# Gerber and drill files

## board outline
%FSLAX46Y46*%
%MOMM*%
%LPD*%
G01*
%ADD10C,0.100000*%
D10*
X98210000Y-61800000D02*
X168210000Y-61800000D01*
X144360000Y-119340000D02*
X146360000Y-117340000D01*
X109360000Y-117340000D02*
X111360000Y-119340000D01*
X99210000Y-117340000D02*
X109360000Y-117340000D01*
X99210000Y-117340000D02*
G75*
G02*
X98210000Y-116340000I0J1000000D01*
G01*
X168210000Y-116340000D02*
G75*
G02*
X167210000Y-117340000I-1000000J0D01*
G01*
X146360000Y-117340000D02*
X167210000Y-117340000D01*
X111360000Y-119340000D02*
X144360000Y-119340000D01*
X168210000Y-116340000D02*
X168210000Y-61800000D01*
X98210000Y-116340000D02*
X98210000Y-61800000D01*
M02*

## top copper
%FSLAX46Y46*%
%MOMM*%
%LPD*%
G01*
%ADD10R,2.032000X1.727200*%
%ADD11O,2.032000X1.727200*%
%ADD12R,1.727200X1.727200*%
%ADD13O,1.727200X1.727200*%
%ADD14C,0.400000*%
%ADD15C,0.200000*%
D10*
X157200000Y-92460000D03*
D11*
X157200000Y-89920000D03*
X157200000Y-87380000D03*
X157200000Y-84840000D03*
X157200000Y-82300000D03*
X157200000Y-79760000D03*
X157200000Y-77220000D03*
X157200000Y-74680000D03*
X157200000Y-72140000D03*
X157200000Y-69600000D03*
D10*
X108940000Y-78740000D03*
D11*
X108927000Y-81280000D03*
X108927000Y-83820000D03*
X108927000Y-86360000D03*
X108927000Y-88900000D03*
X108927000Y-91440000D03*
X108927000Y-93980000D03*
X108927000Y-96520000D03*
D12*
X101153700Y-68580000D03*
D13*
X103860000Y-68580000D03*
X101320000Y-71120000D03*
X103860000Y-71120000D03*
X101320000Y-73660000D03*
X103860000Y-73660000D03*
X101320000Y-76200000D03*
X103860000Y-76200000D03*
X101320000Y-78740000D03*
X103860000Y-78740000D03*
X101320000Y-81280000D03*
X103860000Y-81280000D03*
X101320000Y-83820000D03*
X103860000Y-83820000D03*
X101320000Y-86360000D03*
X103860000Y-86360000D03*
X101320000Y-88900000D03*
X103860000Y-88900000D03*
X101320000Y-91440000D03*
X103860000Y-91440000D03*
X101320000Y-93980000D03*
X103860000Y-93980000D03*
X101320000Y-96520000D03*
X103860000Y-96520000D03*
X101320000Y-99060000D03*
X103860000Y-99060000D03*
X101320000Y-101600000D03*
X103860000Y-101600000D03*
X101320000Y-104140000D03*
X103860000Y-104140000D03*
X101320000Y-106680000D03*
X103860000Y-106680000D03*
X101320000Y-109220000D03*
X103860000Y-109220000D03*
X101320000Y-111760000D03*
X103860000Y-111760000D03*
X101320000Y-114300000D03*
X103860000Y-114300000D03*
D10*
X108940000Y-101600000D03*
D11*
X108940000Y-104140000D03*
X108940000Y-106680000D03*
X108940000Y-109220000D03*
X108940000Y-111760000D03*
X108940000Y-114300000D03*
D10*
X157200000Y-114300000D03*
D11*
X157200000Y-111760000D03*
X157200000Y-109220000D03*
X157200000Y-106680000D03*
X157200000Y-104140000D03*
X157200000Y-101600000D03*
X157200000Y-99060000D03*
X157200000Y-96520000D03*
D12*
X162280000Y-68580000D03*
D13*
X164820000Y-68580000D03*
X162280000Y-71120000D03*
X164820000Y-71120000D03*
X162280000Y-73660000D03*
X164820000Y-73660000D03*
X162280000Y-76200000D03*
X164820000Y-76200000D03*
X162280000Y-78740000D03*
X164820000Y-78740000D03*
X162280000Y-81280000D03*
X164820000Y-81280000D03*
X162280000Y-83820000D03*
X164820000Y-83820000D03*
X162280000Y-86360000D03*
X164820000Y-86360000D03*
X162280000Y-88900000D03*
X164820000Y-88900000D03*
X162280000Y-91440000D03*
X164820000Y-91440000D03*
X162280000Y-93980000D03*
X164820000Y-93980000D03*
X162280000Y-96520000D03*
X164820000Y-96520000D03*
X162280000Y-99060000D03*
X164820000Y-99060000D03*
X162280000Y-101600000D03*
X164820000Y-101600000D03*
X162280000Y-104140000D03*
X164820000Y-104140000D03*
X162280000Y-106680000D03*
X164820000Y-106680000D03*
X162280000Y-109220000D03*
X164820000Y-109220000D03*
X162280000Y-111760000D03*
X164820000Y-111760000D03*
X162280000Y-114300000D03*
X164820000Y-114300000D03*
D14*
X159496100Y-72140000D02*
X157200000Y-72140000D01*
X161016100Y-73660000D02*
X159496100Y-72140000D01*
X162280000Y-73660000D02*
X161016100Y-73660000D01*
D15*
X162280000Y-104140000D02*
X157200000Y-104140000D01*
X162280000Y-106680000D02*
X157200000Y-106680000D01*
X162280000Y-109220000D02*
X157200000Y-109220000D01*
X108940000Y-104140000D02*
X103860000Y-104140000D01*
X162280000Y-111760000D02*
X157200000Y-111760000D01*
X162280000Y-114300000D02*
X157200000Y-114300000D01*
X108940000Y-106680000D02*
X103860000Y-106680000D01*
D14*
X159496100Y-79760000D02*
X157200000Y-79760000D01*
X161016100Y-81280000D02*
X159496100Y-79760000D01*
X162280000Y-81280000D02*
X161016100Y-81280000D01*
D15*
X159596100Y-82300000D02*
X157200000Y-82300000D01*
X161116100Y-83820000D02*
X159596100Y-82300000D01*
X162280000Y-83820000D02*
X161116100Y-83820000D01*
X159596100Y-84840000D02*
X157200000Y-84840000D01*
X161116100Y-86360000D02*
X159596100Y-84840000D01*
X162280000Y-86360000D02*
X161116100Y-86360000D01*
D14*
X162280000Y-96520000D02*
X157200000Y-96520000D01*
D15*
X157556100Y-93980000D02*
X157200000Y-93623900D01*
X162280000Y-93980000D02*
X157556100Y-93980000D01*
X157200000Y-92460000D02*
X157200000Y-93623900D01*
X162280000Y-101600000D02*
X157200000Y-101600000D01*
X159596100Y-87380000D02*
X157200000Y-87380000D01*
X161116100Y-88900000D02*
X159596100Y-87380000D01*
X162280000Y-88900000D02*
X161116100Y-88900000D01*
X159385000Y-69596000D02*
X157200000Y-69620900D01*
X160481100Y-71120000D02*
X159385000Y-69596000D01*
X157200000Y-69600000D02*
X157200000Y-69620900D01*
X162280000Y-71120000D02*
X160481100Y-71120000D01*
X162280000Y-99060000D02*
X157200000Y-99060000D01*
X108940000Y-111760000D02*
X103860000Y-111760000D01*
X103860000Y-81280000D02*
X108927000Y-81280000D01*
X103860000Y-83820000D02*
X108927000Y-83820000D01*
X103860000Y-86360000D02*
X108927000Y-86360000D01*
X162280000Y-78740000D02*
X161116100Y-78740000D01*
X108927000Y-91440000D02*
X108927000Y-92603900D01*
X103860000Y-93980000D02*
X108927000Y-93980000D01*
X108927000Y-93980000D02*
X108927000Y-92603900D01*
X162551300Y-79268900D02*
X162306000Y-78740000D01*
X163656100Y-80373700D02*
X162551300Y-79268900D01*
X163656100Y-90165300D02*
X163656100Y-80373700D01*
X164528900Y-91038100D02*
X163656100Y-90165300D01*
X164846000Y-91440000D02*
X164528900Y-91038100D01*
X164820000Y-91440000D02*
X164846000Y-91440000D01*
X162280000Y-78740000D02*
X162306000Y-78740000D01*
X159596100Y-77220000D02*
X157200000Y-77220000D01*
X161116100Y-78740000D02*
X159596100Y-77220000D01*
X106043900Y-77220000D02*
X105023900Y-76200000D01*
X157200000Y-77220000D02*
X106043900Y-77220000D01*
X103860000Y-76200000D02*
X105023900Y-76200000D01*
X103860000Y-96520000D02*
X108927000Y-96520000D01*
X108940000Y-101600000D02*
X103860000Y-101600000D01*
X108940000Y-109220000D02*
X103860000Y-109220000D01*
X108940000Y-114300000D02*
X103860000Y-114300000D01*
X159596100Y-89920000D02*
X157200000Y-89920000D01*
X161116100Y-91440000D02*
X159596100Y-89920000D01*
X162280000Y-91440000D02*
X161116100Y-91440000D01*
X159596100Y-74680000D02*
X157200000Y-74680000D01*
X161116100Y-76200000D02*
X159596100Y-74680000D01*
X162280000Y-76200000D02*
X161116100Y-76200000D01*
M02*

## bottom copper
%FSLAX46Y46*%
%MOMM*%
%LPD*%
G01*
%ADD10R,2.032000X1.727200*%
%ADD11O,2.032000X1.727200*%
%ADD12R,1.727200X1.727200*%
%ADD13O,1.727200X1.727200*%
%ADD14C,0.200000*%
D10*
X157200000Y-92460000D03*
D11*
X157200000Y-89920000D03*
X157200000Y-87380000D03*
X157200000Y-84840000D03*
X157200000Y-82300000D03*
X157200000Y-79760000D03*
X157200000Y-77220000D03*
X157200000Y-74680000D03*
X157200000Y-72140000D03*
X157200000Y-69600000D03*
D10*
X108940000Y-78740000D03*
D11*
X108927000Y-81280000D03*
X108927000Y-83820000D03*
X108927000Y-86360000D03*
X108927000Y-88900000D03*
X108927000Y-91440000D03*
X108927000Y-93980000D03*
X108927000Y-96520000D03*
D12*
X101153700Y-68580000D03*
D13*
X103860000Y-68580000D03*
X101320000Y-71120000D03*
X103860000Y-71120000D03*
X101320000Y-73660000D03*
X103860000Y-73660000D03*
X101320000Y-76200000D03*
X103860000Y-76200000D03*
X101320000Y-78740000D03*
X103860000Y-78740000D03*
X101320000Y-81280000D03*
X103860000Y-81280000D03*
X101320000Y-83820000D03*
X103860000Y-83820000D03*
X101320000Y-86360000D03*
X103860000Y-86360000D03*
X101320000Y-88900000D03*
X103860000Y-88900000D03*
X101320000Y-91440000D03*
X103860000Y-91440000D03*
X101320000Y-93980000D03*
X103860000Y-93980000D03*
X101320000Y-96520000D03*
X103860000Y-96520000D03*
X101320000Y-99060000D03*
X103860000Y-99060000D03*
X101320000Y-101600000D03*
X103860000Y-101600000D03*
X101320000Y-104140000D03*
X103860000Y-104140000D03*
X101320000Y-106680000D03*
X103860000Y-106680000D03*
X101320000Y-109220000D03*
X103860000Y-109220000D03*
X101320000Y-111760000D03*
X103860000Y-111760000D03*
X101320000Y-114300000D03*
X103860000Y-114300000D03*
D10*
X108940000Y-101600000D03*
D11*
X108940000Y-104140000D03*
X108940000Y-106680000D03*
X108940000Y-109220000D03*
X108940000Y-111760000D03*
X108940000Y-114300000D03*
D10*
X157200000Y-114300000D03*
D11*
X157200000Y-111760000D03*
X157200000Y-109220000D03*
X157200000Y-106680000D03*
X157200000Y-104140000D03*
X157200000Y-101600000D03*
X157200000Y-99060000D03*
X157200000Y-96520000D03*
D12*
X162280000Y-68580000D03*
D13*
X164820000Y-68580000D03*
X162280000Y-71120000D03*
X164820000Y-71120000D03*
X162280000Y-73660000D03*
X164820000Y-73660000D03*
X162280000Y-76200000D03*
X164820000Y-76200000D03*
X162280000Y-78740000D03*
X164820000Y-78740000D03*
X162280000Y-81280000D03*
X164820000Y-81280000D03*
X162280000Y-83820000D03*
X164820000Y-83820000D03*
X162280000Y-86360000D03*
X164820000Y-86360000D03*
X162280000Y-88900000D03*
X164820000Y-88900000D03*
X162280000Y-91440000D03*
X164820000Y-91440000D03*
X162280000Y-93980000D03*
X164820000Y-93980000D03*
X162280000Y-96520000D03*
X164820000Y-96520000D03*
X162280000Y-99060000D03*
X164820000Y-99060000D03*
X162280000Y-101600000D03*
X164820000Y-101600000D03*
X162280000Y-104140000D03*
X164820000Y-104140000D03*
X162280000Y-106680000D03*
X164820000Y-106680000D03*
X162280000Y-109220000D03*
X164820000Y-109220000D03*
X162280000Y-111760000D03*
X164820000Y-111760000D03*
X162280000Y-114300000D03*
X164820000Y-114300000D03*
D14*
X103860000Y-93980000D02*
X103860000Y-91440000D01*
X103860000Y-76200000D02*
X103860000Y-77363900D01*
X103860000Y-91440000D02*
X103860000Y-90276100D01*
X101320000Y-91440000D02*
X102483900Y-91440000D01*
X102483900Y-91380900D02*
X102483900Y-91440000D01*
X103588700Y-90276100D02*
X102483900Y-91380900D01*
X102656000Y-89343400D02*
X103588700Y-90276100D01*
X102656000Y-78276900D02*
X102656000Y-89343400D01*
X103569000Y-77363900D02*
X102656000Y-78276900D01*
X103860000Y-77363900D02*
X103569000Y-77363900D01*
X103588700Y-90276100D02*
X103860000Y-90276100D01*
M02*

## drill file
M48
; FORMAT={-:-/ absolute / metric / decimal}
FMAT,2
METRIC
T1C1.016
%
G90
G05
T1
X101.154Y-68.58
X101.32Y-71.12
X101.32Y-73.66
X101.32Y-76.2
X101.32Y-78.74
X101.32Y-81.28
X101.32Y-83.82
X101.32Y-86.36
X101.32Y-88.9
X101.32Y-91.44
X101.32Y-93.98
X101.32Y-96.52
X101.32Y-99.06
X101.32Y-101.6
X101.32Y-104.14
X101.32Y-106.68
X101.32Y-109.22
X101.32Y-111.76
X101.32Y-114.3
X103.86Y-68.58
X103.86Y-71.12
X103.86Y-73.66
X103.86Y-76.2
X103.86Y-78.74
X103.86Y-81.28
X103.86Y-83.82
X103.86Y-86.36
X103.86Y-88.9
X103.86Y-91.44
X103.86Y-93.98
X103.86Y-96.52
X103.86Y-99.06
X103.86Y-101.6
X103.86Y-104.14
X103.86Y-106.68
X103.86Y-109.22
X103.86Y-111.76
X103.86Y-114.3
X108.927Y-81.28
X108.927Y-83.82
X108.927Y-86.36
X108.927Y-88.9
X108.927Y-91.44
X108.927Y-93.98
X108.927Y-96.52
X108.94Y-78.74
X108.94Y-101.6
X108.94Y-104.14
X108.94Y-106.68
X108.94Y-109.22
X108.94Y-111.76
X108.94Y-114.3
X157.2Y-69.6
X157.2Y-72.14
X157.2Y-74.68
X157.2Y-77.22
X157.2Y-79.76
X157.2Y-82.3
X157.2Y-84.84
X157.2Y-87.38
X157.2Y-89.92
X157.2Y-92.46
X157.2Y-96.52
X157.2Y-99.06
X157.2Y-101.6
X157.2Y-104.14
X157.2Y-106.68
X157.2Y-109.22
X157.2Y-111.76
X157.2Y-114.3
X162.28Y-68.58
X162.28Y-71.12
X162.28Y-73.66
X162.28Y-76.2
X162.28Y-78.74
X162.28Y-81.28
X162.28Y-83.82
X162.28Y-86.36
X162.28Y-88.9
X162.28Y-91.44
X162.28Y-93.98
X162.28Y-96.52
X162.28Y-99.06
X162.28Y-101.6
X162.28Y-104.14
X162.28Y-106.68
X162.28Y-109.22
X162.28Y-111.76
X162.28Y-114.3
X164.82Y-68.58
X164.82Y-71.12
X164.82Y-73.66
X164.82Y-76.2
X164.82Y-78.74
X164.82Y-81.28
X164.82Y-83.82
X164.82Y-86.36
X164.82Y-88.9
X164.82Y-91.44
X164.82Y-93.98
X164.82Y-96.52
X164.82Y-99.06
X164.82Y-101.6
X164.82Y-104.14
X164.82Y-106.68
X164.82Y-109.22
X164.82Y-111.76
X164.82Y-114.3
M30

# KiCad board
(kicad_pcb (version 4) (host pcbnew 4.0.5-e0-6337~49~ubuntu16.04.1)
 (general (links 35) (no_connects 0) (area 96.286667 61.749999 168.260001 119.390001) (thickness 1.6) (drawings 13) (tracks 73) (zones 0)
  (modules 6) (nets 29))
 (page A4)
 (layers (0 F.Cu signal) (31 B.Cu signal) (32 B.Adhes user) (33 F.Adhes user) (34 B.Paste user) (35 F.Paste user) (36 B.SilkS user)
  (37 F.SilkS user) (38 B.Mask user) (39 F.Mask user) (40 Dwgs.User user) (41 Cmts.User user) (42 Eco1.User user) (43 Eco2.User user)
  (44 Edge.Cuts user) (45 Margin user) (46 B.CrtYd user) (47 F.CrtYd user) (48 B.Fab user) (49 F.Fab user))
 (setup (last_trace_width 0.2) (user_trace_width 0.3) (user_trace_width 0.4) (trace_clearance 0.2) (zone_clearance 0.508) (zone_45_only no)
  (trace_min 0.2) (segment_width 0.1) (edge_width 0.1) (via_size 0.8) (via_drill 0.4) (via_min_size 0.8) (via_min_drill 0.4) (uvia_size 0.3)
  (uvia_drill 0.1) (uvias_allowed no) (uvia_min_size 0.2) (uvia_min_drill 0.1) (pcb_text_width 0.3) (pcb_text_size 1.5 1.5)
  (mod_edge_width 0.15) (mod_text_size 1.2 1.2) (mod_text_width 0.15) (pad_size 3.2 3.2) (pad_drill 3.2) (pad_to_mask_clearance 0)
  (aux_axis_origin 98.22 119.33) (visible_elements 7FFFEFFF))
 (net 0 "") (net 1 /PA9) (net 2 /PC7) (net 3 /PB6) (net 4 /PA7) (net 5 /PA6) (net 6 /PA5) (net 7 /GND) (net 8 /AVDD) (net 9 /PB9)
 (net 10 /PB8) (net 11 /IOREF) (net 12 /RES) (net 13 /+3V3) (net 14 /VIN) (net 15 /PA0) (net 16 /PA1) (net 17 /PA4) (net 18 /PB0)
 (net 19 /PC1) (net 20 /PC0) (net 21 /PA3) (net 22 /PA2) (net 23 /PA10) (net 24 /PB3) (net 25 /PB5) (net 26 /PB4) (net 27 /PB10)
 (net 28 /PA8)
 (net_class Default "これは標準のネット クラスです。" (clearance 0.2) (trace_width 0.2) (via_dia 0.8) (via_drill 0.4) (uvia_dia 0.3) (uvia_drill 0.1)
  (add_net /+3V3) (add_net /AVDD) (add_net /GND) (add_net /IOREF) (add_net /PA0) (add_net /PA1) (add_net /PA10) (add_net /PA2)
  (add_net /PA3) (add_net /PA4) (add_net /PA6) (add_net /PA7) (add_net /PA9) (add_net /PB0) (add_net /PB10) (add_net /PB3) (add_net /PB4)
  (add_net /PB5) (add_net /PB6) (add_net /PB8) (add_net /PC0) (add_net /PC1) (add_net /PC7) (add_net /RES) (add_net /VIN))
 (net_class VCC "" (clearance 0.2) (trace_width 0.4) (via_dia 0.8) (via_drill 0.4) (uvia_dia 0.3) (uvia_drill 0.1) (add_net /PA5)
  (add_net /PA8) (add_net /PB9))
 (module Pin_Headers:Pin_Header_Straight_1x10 (layer F.Cu) (at 157.2 92.46 180)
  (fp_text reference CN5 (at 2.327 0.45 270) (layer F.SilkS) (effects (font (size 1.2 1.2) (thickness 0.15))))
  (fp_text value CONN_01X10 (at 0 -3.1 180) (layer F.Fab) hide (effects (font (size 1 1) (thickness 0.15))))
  (pad 1 thru_hole rect (at 0 0 180) (size 2.032 1.7272) (drill 1.016) (layers *.Cu *.Mask F.SilkS) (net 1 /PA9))
  (pad 2 thru_hole oval (at 0 2.54 180) (size 2.032 1.7272) (drill 1.016) (layers *.Cu *.Mask F.SilkS) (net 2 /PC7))
  (pad 3 thru_hole oval (at 0 5.08 180) (size 2.032 1.7272) (drill 1.016) (layers *.Cu *.Mask F.SilkS) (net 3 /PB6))
  (pad 4 thru_hole oval (at 0 7.62 180) (size 2.032 1.7272) (drill 1.016) (layers *.Cu *.Mask F.SilkS) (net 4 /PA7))
  (pad 5 thru_hole oval (at 0 10.16 180) (size 2.032 1.7272) (drill 1.016) (layers *.Cu *.Mask F.SilkS) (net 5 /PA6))
  (pad 6 thru_hole oval (at 0 12.7 180) (size 2.032 1.7272) (drill 1.016) (layers *.Cu *.Mask F.SilkS) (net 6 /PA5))
  (pad 7 thru_hole oval (at 0 15.24 180) (size 2.032 1.7272) (drill 1.016) (layers *.Cu *.Mask F.SilkS) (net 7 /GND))
  (pad 8 thru_hole oval (at 0 17.78 180) (size 2.032 1.7272) (drill 1.016) (layers *.Cu *.Mask F.SilkS) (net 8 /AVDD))
  (pad 9 thru_hole oval (at 0 20.32 180) (size 2.032 1.7272) (drill 1.016) (layers *.Cu *.Mask F.SilkS) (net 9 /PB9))
  (pad 10 thru_hole oval (at 0 22.86 180) (size 2.032 1.7272) (drill 1.016) (layers *.Cu *.Mask F.SilkS) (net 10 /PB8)))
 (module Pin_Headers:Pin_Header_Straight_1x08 (layer F.Cu) (at 108.927 78.74)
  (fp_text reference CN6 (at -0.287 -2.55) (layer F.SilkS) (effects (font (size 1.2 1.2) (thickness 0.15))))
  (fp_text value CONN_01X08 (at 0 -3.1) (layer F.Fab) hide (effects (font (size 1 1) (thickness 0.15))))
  (pad 1 thru_hole rect (at 0.013 0) (size 2.032 1.7272) (drill 1.016) (layers *.Cu *.Mask F.SilkS))
  (pad 2 thru_hole oval (at 0 2.54) (size 2.032 1.7272) (drill 1.016) (layers *.Cu *.Mask F.SilkS) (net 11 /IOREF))
  (pad 3 thru_hole oval (at 0 5.08) (size 2.032 1.7272) (drill 1.016) (layers *.Cu *.Mask F.SilkS) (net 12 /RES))
  (pad 4 thru_hole oval (at 0 7.62) (size 2.032 1.7272) (drill 1.016) (layers *.Cu *.Mask F.SilkS) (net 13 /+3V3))
  (pad 5 thru_hole oval (at 0 10.16) (size 2.032 1.7272) (drill 1.016) (layers *.Cu *.Mask F.SilkS))
  (pad 6 thru_hole oval (at 0 12.7) (size 2.032 1.7272) (drill 1.016) (layers *.Cu *.Mask F.SilkS) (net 7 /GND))
  (pad 7 thru_hole oval (at 0 15.24) (size 2.032 1.7272) (drill 1.016) (layers *.Cu *.Mask F.SilkS) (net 7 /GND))
  (pad 8 thru_hole oval (at 0 17.78) (size 2.032 1.7272) (drill 1.016) (layers *.Cu *.Mask F.SilkS) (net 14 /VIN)))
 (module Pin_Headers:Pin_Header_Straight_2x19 (layer F.Cu) (at 101.32 68.58)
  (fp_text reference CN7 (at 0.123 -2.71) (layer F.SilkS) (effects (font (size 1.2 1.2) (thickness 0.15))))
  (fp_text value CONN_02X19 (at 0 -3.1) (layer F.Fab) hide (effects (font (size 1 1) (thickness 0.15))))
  (pad 1 thru_hole rect (at -0.1663 0) (size 1.7272 1.7272) (drill 1.016) (layers *.Cu *.Mask F.SilkS))
  (pad 2 thru_hole oval (at 2.54 0) (size 1.7272 1.7272) (drill 1.016) (layers *.Cu *.Mask F.SilkS))
  (pad 3 thru_hole oval (at 0 2.54) (size 1.7272 1.7272) (drill 1.016) (layers *.Cu *.Mask F.SilkS))
  (pad 4 thru_hole oval (at 2.54 2.54) (size 1.7272 1.7272) (drill 1.016) (layers *.Cu *.Mask F.SilkS))
  (pad 5 thru_hole oval (at 0 5.08) (size 1.7272 1.7272) (drill 1.016) (layers *.Cu *.Mask F.SilkS))
  (pad 6 thru_hole oval (at 2.54 5.08) (size 1.7272 1.7272) (drill 1.016) (layers *.Cu *.Mask F.SilkS))
  (pad 7 thru_hole oval (at 0 7.62) (size 1.7272 1.7272) (drill 1.016) (layers *.Cu *.Mask F.SilkS))
  (pad 8 thru_hole oval (at 2.54 7.62) (size 1.7272 1.7272) (drill 1.016) (layers *.Cu *.Mask F.SilkS) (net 7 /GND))
  (pad 9 thru_hole oval (at 0 10.16) (size 1.7272 1.7272) (drill 1.016) (layers *.Cu *.Mask F.SilkS))
  (pad 10 thru_hole oval (at 2.54 10.16) (size 1.7272 1.7272) (drill 1.016) (layers *.Cu *.Mask F.SilkS))
  (pad 11 thru_hole oval (at 0 12.7) (size 1.7272 1.7272) (drill 1.016) (layers *.Cu *.Mask F.SilkS))
  (pad 12 thru_hole oval (at 2.54 12.7) (size 1.7272 1.7272) (drill 1.016) (layers *.Cu *.Mask F.SilkS) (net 11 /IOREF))
  (pad 13 thru_hole oval (at 0 15.24) (size 1.7272 1.7272) (drill 1.016) (layers *.Cu *.Mask F.SilkS))
  (pad 14 thru_hole oval (at 2.54 15.24) (size 1.7272 1.7272) (drill 1.016) (layers *.Cu *.Mask F.SilkS) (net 12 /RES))
  (pad 15 thru_hole oval (at 0 17.78) (size 1.7272 1.7272) (drill 1.016) (layers *.Cu *.Mask F.SilkS))
  (pad 16 thru_hole oval (at 2.54 17.78) (size 1.7272 1.7272) (drill 1.016) (layers *.Cu *.Mask F.SilkS) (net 13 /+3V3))
  (pad 17 thru_hole oval (at 0 20.32) (size 1.7272 1.7272) (drill 1.016) (layers *.Cu *.Mask F.SilkS))
  (pad 18 thru_hole oval (at 2.54 20.32) (size 1.7272 1.7272) (drill 1.016) (layers *.Cu *.Mask F.SilkS))
  (pad 19 thru_hole oval (at 0 22.86) (size 1.7272 1.7272) (drill 1.016) (layers *.Cu *.Mask F.SilkS) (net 7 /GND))
  (pad 20 thru_hole oval (at 2.54 22.86) (size 1.7272 1.7272) (drill 1.016) (layers *.Cu *.Mask F.SilkS) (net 7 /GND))
  (pad 21 thru_hole oval (at 0 25.4) (size 1.7272 1.7272) (drill 1.016) (layers *.Cu *.Mask F.SilkS))
  (pad 22 thru_hole oval (at 2.54 25.4) (size 1.7272 1.7272) (drill 1.016) (layers *.Cu *.Mask F.SilkS) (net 7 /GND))
  (pad 23 thru_hole oval (at 0 27.94) (size 1.7272 1.7272) (drill 1.016) (layers *.Cu *.Mask F.SilkS))
  (pad 24 thru_hole oval (at 2.54 27.94) (size 1.7272 1.7272) (drill 1.016) (layers *.Cu *.Mask F.SilkS) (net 14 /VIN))
  (pad 25 thru_hole oval (at 0 30.48) (size 1.7272 1.7272) (drill 1.016) (layers *.Cu *.Mask F.SilkS))
  (pad 26 thru_hole oval (at 2.54 30.48) (size 1.7272 1.7272) (drill 1.016) (layers *.Cu *.Mask F.SilkS))
  (pad 27 thru_hole oval (at 0 33.02) (size 1.7272 1.7272) (drill 1.016) (layers *.Cu *.Mask F.SilkS))
  (pad 28 thru_hole oval (at 2.54 33.02) (size 1.7272 1.7272) (drill 1.016) (layers *.Cu *.Mask F.SilkS) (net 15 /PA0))
  (pad 29 thru_hole oval (at 0 35.56) (size 1.7272 1.7272) (drill 1.016) (layers *.Cu *.Mask F.SilkS))
  (pad 30 thru_hole oval (at 2.54 35.56) (size 1.7272 1.7272) (drill 1.016) (layers *.Cu *.Mask F.SilkS) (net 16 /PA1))
  (pad 31 thru_hole oval (at 0 38.1) (size 1.7272 1.7272) (drill 1.016) (layers *.Cu *.Mask F.SilkS))
  (pad 32 thru_hole oval (at 2.54 38.1) (size 1.7272 1.7272) (drill 1.016) (layers *.Cu *.Mask F.SilkS) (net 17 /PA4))
  (pad 33 thru_hole oval (at 0 40.64) (size 1.7272 1.7272) (drill 1.016) (layers *.Cu *.Mask F.SilkS))
  (pad 34 thru_hole oval (at 2.54 40.64) (size 1.7272 1.7272) (drill 1.016) (layers *.Cu *.Mask F.SilkS) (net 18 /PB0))
  (pad 35 thru_hole oval (at 0 43.18) (size 1.7272 1.7272) (drill 1.016) (layers *.Cu *.Mask F.SilkS))
  (pad 36 thru_hole oval (at 2.54 43.18) (size 1.7272 1.7272) (drill 1.016) (layers *.Cu *.Mask F.SilkS) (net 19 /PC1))
  (pad 37 thru_hole oval (at 0 45.72) (size 1.7272 1.7272) (drill 1.016) (layers *.Cu *.Mask F.SilkS))
  (pad 38 thru_hole oval (at 2.54 45.72) (size 1.7272 1.7272) (drill 1.016) (layers *.Cu *.Mask F.SilkS) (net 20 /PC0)))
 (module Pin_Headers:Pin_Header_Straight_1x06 (layer F.Cu) (at 108.94 101.6)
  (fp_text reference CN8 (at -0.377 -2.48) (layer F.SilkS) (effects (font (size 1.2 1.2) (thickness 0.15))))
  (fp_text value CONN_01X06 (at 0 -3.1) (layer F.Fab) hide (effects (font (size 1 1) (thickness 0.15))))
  (pad 1 thru_hole rect (at 0 0) (size 2.032 1.7272) (drill 1.016) (layers *.Cu *.Mask F.SilkS) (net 15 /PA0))
  (pad 2 thru_hole oval (at 0 2.54) (size 2.032 1.7272) (drill 1.016) (layers *.Cu *.Mask F.SilkS) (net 16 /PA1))
  (pad 3 thru_hole oval (at 0 5.08) (size 2.032 1.7272) (drill 1.016) (layers *.Cu *.Mask F.SilkS) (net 17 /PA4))
  (pad 4 thru_hole oval (at 0 7.62) (size 2.032 1.7272) (drill 1.016) (layers *.Cu *.Mask F.SilkS) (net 18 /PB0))
  (pad 5 thru_hole oval (at 0 10.16) (size 2.032 1.7272) (drill 1.016) (layers *.Cu *.Mask F.SilkS) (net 19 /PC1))
  (pad 6 thru_hole oval (at 0 12.7) (size 2.032 1.7272) (drill 1.016) (layers *.Cu *.Mask F.SilkS) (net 20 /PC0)))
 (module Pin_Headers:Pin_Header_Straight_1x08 (layer F.Cu) (at 157.2 114.3 180)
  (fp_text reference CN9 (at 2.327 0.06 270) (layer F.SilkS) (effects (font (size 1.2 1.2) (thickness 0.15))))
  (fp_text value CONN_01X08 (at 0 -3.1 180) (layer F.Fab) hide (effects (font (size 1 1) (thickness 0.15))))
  (pad 1 thru_hole rect (at 0 0 180) (size 2.032 1.7272) (drill 1.016) (layers *.Cu *.Mask F.SilkS) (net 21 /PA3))
  (pad 2 thru_hole oval (at 0 2.54 180) (size 2.032 1.7272) (drill 1.016) (layers *.Cu *.Mask F.SilkS) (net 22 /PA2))
  (pad 3 thru_hole oval (at 0 5.08 180) (size 2.032 1.7272) (drill 1.016) (layers *.Cu *.Mask F.SilkS) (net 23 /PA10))
  (pad 4 thru_hole oval (at 0 7.62 180) (size 2.032 1.7272) (drill 1.016) (layers *.Cu *.Mask F.SilkS) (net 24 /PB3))
  (pad 5 thru_hole oval (at 0 10.16 180) (size 2.032 1.7272) (drill 1.016) (layers *.Cu *.Mask F.SilkS) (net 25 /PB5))
  (pad 6 thru_hole oval (at 0 12.7 180) (size 2.032 1.7272) (drill 1.016) (layers *.Cu *.Mask F.SilkS) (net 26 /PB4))
  (pad 7 thru_hole oval (at 0 15.24 180) (size 2.032 1.7272) (drill 1.016) (layers *.Cu *.Mask F.SilkS) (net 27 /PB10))
  (pad 8 thru_hole oval (at 0 17.78 180) (size 2.032 1.7272) (drill 1.016) (layers *.Cu *.Mask F.SilkS) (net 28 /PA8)))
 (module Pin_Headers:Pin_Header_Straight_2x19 (layer F.Cu) (at 162.28 68.58)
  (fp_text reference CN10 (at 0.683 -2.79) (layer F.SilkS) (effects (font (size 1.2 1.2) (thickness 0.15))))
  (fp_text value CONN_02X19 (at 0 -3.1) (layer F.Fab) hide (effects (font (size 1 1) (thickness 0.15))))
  (pad 1 thru_hole rect (at 0 0) (size 1.7272 1.7272) (drill 1.016) (layers *.Cu *.Mask F.SilkS))
  (pad 2 thru_hole oval (at 2.54 0) (size 1.7272 1.7272) (drill 1.016) (layers *.Cu *.Mask F.SilkS))
  (pad 3 thru_hole oval (at 0 2.54) (size 1.7272 1.7272) (drill 1.016) (layers *.Cu *.Mask F.SilkS) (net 10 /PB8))
  (pad 4 thru_hole oval (at 2.54 2.54) (size 1.7272 1.7272) (drill 1.016) (layers *.Cu *.Mask F.SilkS))
  (pad 5 thru_hole oval (at 0 5.08) (size 1.7272 1.7272) (drill 1.016) (layers *.Cu *.Mask F.SilkS) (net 9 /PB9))
  (pad 6 thru_hole oval (at 2.54 5.08) (size 1.7272 1.7272) (drill 1.016) (layers *.Cu *.Mask F.SilkS))
  (pad 7 thru_hole oval (at 0 7.62) (size 1.7272 1.7272) (drill 1.016) (layers *.Cu *.Mask F.SilkS) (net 8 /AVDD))
  (pad 8 thru_hole oval (at 2.54 7.62) (size 1.7272 1.7272) (drill 1.016) (layers *.Cu *.Mask F.SilkS))
  (pad 9 thru_hole oval (at 0 10.16) (size 1.7272 1.7272) (drill 1.016) (layers *.Cu *.Mask F.SilkS) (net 7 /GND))
  (pad 10 thru_hole oval (at 2.54 10.16) (size 1.7272 1.7272) (drill 1.016) (layers *.Cu *.Mask F.SilkS))
  (pad 11 thru_hole oval (at 0 12.7) (size 1.7272 1.7272) (drill 1.016) (layers *.Cu *.Mask F.SilkS) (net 6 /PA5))
  (pad 12 thru_hole oval (at 2.54 12.7) (size 1.7272 1.7272) (drill 1.016) (layers *.Cu *.Mask F.SilkS))
  (pad 13 thru_hole oval (at 0 15.24) (size 1.7272 1.7272) (drill 1.016) (layers *.Cu *.Mask F.SilkS) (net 5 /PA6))
  (pad 14 thru_hole oval (at 2.54 15.24) (size 1.7272 1.7272) (drill 1.016) (layers *.Cu *.Mask F.SilkS))
  (pad 15 thru_hole oval (at 0 17.78) (size 1.7272 1.7272) (drill 1.016) (layers *.Cu *.Mask F.SilkS) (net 4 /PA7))
  (pad 16 thru_hole oval (at 2.54 17.78) (size 1.7272 1.7272) (drill 1.016) (layers *.Cu *.Mask F.SilkS))
  (pad 17 thru_hole oval (at 0 20.32) (size 1.7272 1.7272) (drill 1.016) (layers *.Cu *.Mask F.SilkS) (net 3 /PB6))
  (pad 18 thru_hole oval (at 2.54 20.32) (size 1.7272 1.7272) (drill 1.016) (layers *.Cu *.Mask F.SilkS))
  (pad 19 thru_hole oval (at 0 22.86) (size 1.7272 1.7272) (drill 1.016) (layers *.Cu *.Mask F.SilkS) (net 2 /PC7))
  (pad 20 thru_hole oval (at 2.54 22.86) (size 1.7272 1.7272) (drill 1.016) (layers *.Cu *.Mask F.SilkS) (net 7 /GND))
  (pad 21 thru_hole oval (at 0 25.4) (size 1.7272 1.7272) (drill 1.016) (layers *.Cu *.Mask F.SilkS) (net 1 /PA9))
  (pad 22 thru_hole oval (at 2.54 25.4) (size 1.7272 1.7272) (drill 1.016) (layers *.Cu *.Mask F.SilkS))
  (pad 23 thru_hole oval (at 0 27.94) (size 1.7272 1.7272) (drill 1.016) (layers *.Cu *.Mask F.SilkS) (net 28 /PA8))
  (pad 24 thru_hole oval (at 2.54 27.94) (size 1.7272 1.7272) (drill 1.016) (layers *.Cu *.Mask F.SilkS))
  (pad 25 thru_hole oval (at 0 30.48) (size 1.7272 1.7272) (drill 1.016) (layers *.Cu *.Mask F.SilkS) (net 27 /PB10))
  (pad 26 thru_hole oval (at 2.54 30.48) (size 1.7272 1.7272) (drill 1.016) (layers *.Cu *.Mask F.SilkS))
  (pad 27 thru_hole oval (at 0 33.02) (size 1.7272 1.7272) (drill 1.016) (layers *.Cu *.Mask F.SilkS) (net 26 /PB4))
  (pad 28 thru_hole oval (at 2.54 33.02) (size 1.7272 1.7272) (drill 1.016) (layers *.Cu *.Mask F.SilkS))
  (pad 29 thru_hole oval (at 0 35.56) (size 1.7272 1.7272) (drill 1.016) (layers *.Cu *.Mask F.SilkS) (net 25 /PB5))
  (pad 30 thru_hole oval (at 2.54 35.56) (size 1.7272 1.7272) (drill 1.016) (layers *.Cu *.Mask F.SilkS))
  (pad 31 thru_hole oval (at 0 38.1) (size 1.7272 1.7272) (drill 1.016) (layers *.Cu *.Mask F.SilkS) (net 24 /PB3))
  (pad 32 thru_hole oval (at 2.54 38.1) (size 1.7272 1.7272) (drill 1.016) (layers *.Cu *.Mask F.SilkS))
  (pad 33 thru_hole oval (at 0 40.64) (size 1.7272 1.7272) (drill 1.016) (layers *.Cu *.Mask F.SilkS) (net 23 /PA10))
  (pad 34 thru_hole oval (at 2.54 40.64) (size 1.7272 1.7272) (drill 1.016) (layers *.Cu *.Mask F.SilkS))
  (pad 35 thru_hole oval (at 0 43.18) (size 1.7272 1.7272) (drill 1.016) (layers *.Cu *.Mask F.SilkS) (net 22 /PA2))
  (pad 36 thru_hole oval (at 2.54 43.18) (size 1.7272 1.7272) (drill 1.016) (layers *.Cu *.Mask F.SilkS))
  (pad 37 thru_hole oval (at 0 45.72) (size 1.7272 1.7272) (drill 1.016) (layers *.Cu *.Mask F.SilkS) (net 21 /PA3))
  (pad 38 thru_hole oval (at 2.54 45.72) (size 1.7272 1.7272) (drill 1.016) (layers *.Cu *.Mask F.SilkS)))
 (gr_line (start 98.21 61.8) (end 168.21 61.8) (angle 90) (layer Edge.Cuts) (width 0.1))
 (gr_line (start 144.36 119.34) (end 146.36 117.34) (angle 90) (layer Edge.Cuts) (width 0.1))
 (gr_line (start 109.36 117.34) (end 111.36 119.34) (angle 90) (layer Edge.Cuts) (width 0.1))
 (gr_line (start 99.21 117.34) (end 109.36 117.34) (angle 90) (layer Edge.Cuts) (width 0.1))
 (gr_arc (start 99.21 116.34) (end 99.21 117.34) (angle 90) (layer Edge.Cuts) (width 0.1))
 (gr_arc (start 167.21 116.34) (end 168.21 116.34) (angle 90) (layer Edge.Cuts) (width 0.1))
 (gr_line (start 146.36 117.34) (end 167.21 117.34) (angle 90) (layer Edge.Cuts) (width 0.1))
 (gr_line (start 111.36 119.34) (end 144.36 119.34) (angle 90) (layer Edge.Cuts) (width 0.1))
 (gr_line (start 168.21 116.34) (end 168.21 61.8) (angle 90) (layer Edge.Cuts) (width 0.1))
 (gr_line (start 98.21 116.34) (end 98.21 61.8) (angle 90) (layer Edge.Cuts) (width 0.1))
 (segment (start 159.4961 72.14) (end 157.2 72.14) (width 0.4) (layer F.Cu) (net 9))
 (segment (start 161.0161 73.66) (end 159.4961 72.14) (width 0.4) (layer F.Cu) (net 9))
 (segment (start 162.28 73.66) (end 161.0161 73.66) (width 0.4) (layer F.Cu) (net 9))
 (segment (start 162.28 104.14) (end 157.2 104.14) (width 0.2) (layer F.Cu) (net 25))
 (segment (start 162.28 106.68) (end 157.2 106.68) (width 0.2) (layer F.Cu) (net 24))
 (segment (start 162.28 109.22) (end 157.2 109.22) (width 0.2) (layer F.Cu) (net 23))
 (segment (start 108.94 104.14) (end 103.86 104.14) (width 0.2) (layer F.Cu) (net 16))
 (segment (start 162.28 111.76) (end 157.2 111.76) (width 0.2) (layer F.Cu) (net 22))
 (segment (start 162.28 114.3) (end 157.2 114.3) (width 0.2) (layer F.Cu) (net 21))
 (segment (start 108.94 106.68) (end 103.86 106.68) (width 0.2) (layer F.Cu) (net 17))
 (segment (start 159.4961 79.76) (end 157.2 79.76) (width 0.4) (layer F.Cu) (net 6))
 (segment (start 161.0161 81.28) (end 159.4961 79.76) (width 0.4) (layer F.Cu) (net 6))
 (segment (start 162.28 81.28) (end 161.0161 81.28) (width 0.4) (layer F.Cu) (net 6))
 (segment (start 159.5961 82.3) (end 157.2 82.3) (width 0.2) (layer F.Cu) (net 5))
 (segment (start 161.1161 83.82) (end 159.5961 82.3) (width 0.2) (layer F.Cu) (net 5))
 (segment (start 162.28 83.82) (end 161.1161 83.82) (width 0.2) (layer F.Cu) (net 5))
 (segment (start 159.5961 84.84) (end 157.2 84.84) (width 0.2) (layer F.Cu) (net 4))
 (segment (start 161.1161 86.36) (end 159.5961 84.84) (width 0.2) (layer F.Cu) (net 4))
 (segment (start 162.28 86.36) (end 161.1161 86.36) (width 0.2) (layer F.Cu) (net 4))
 (segment (start 162.28 96.52) (end 157.2 96.52) (width 0.4) (layer F.Cu) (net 28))
 (segment (start 157.5561 93.98) (end 157.2 93.6239) (width 0.2) (layer F.Cu) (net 1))
 (segment (start 162.28 93.98) (end 157.5561 93.98) (width 0.2) (layer F.Cu) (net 1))
 (segment (start 157.2 92.46) (end 157.2 93.6239) (width 0.2) (layer F.Cu) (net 1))
 (segment (start 162.28 101.6) (end 157.2 101.6) (width 0.2) (layer F.Cu) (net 26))
 (segment (start 159.5961 87.38) (end 157.2 87.38) (width 0.2) (layer F.Cu) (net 3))
 (segment (start 161.1161 88.9) (end 159.5961 87.38) (width 0.2) (layer F.Cu) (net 3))
 (segment (start 162.28 88.9) (end 161.1161 88.9) (width 0.2) (layer F.Cu) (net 3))
 (segment (start 159.385 69.596) (end 157.2 69.6209) (width 0.2) (layer F.Cu) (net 10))
 (segment (start 160.4811 71.12) (end 159.385 69.596) (width 0.2) (layer F.Cu) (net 10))
 (segment (start 157.2 69.6) (end 157.2 69.6209) (width 0.2) (layer F.Cu) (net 10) (status 400000))
 (segment (start 162.28 71.12) (end 160.4811 71.12) (width 0.2) (layer F.Cu) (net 10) (status 400000))
 (segment (start 162.28 99.06) (end 157.2 99.06) (width 0.2) (layer F.Cu) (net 27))
 (segment (start 108.94 111.76) (end 103.86 111.76) (width 0.2) (layer F.Cu) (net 19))
 (segment (start 103.86 81.28) (end 108.927 81.28) (width 0.2) (layer F.Cu) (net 11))
 (segment (start 103.86 83.82) (end 108.927 83.82) (width 0.2) (layer F.Cu) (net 12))
 (segment (start 103.86 86.36) (end 108.927 86.36) (width 0.2) (layer F.Cu) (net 13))
 (segment (start 103.86 93.98) (end 103.86 91.44) (width 0.2) (layer B.Cu) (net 7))
 (segment (start 103.86 76.2) (end 103.86 77.3639) (width 0.2) (layer B.Cu) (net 7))
 (segment (start 103.86 91.44) (end 103.86 90.2761) (width 0.2) (layer B.Cu) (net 7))
 (segment (start 162.28 78.74) (end 161.1161 78.74) (width 0.2) (layer F.Cu) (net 7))
 (segment (start 101.32 91.44) (end 102.4839 91.44) (width 0.2) (layer B.Cu) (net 7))
 (segment (start 102.4839 91.3809) (end 102.4839 91.44) (width 0.2) (layer B.Cu) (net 7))
 (segment (start 103.5887 90.2761) (end 102.4839 91.3809) (width 0.2) (layer B.Cu) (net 7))
 (segment (start 102.656 89.3434) (end 103.5887 90.2761) (width 0.2) (layer B.Cu) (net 7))
 (segment (start 102.656 78.2769) (end 102.656 89.3434) (width 0.2) (layer B.Cu) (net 7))
 (segment (start 103.569 77.3639) (end 102.656 78.2769) (width 0.2) (layer B.Cu) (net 7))
 (segment (start 103.86 77.3639) (end 103.569 77.3639) (width 0.2) (layer B.Cu) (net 7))
 (segment (start 103.5887 90.2761) (end 103.86 90.2761) (width 0.2) (layer B.Cu) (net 7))
 (segment (start 108.927 91.44) (end 108.927 92.6039) (width 0.2) (layer F.Cu) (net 7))
 (segment (start 103.86 93.98) (end 108.927 93.98) (width 0.2) (layer F.Cu) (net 7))
 (segment (start 108.927 93.98) (end 108.927 92.6039) (width 0.2) (layer F.Cu) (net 7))
 (segment (start 162.5513 79.2689) (end 162.306 78.74) (width 0.2) (layer F.Cu) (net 7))
 (segment (start 163.6561 80.3737) (end 162.5513 79.2689) (width 0.2) (layer F.Cu) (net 7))
 (segment (start 163.6561 90.1653) (end 163.6561 80.3737) (width 0.2) (layer F.Cu) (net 7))
 (segment (start 164.5289 91.0381) (end 163.6561 90.1653) (width 0.2) (layer F.Cu) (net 7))
 (segment (start 164.846 91.44) (end 164.5289 91.0381) (width 0.2) (layer F.Cu) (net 7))
 (segment (start 164.82 91.44) (end 164.846 91.44) (width 0.2) (layer F.Cu) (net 7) (status 400000))
 (segment (start 162.28 78.74) (end 162.306 78.74) (width 0.2) (layer F.Cu) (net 7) (status 400000))
 (segment (start 159.5961 77.22) (end 157.2 77.22) (width 0.2) (layer F.Cu) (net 7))
 (segment (start 161.1161 78.74) (end 159.5961 77.22) (width 0.2) (layer F.Cu) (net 7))
 (segment (start 106.0439 77.22) (end 105.0239 76.2) (width 0.2) (layer F.Cu) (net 7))
 (segment (start 157.2 77.22) (end 106.0439 77.22) (width 0.2) (layer F.Cu) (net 7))
 (segment (start 103.86 76.2) (end 105.0239 76.2) (width 0.2) (layer F.Cu) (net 7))
 (segment (start 103.86 96.52) (end 108.927 96.52) (width 0.2) (layer F.Cu) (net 14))
 (segment (start 108.94 101.6) (end 103.86 101.6) (width 0.2) (layer F.Cu) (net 15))
 (segment (start 108.94 109.22) (end 103.86 109.22) (width 0.2) (layer F.Cu) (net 18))
 (segment (start 108.94 114.3) (end 103.86 114.3) (width 0.2) (layer F.Cu) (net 20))
 (segment (start 159.5961 89.92) (end 157.2 89.92) (width 0.2) (layer F.Cu) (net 2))
 (segment (start 161.1161 91.44) (end 159.5961 89.92) (width 0.2) (layer F.Cu) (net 2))
 (segment (start 162.28 91.44) (end 161.1161 91.44) (width 0.2) (layer F.Cu) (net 2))
 (segment (start 159.5961 74.68) (end 157.2 74.68) (width 0.2) (layer F.Cu) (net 8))
 (segment (start 161.1161 76.2) (end 159.5961 74.68) (width 0.2) (layer F.Cu) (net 8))
 (segment (start 162.28 76.2) (end 161.1161 76.2) (width 0.2) (layer F.Cu) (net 8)))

